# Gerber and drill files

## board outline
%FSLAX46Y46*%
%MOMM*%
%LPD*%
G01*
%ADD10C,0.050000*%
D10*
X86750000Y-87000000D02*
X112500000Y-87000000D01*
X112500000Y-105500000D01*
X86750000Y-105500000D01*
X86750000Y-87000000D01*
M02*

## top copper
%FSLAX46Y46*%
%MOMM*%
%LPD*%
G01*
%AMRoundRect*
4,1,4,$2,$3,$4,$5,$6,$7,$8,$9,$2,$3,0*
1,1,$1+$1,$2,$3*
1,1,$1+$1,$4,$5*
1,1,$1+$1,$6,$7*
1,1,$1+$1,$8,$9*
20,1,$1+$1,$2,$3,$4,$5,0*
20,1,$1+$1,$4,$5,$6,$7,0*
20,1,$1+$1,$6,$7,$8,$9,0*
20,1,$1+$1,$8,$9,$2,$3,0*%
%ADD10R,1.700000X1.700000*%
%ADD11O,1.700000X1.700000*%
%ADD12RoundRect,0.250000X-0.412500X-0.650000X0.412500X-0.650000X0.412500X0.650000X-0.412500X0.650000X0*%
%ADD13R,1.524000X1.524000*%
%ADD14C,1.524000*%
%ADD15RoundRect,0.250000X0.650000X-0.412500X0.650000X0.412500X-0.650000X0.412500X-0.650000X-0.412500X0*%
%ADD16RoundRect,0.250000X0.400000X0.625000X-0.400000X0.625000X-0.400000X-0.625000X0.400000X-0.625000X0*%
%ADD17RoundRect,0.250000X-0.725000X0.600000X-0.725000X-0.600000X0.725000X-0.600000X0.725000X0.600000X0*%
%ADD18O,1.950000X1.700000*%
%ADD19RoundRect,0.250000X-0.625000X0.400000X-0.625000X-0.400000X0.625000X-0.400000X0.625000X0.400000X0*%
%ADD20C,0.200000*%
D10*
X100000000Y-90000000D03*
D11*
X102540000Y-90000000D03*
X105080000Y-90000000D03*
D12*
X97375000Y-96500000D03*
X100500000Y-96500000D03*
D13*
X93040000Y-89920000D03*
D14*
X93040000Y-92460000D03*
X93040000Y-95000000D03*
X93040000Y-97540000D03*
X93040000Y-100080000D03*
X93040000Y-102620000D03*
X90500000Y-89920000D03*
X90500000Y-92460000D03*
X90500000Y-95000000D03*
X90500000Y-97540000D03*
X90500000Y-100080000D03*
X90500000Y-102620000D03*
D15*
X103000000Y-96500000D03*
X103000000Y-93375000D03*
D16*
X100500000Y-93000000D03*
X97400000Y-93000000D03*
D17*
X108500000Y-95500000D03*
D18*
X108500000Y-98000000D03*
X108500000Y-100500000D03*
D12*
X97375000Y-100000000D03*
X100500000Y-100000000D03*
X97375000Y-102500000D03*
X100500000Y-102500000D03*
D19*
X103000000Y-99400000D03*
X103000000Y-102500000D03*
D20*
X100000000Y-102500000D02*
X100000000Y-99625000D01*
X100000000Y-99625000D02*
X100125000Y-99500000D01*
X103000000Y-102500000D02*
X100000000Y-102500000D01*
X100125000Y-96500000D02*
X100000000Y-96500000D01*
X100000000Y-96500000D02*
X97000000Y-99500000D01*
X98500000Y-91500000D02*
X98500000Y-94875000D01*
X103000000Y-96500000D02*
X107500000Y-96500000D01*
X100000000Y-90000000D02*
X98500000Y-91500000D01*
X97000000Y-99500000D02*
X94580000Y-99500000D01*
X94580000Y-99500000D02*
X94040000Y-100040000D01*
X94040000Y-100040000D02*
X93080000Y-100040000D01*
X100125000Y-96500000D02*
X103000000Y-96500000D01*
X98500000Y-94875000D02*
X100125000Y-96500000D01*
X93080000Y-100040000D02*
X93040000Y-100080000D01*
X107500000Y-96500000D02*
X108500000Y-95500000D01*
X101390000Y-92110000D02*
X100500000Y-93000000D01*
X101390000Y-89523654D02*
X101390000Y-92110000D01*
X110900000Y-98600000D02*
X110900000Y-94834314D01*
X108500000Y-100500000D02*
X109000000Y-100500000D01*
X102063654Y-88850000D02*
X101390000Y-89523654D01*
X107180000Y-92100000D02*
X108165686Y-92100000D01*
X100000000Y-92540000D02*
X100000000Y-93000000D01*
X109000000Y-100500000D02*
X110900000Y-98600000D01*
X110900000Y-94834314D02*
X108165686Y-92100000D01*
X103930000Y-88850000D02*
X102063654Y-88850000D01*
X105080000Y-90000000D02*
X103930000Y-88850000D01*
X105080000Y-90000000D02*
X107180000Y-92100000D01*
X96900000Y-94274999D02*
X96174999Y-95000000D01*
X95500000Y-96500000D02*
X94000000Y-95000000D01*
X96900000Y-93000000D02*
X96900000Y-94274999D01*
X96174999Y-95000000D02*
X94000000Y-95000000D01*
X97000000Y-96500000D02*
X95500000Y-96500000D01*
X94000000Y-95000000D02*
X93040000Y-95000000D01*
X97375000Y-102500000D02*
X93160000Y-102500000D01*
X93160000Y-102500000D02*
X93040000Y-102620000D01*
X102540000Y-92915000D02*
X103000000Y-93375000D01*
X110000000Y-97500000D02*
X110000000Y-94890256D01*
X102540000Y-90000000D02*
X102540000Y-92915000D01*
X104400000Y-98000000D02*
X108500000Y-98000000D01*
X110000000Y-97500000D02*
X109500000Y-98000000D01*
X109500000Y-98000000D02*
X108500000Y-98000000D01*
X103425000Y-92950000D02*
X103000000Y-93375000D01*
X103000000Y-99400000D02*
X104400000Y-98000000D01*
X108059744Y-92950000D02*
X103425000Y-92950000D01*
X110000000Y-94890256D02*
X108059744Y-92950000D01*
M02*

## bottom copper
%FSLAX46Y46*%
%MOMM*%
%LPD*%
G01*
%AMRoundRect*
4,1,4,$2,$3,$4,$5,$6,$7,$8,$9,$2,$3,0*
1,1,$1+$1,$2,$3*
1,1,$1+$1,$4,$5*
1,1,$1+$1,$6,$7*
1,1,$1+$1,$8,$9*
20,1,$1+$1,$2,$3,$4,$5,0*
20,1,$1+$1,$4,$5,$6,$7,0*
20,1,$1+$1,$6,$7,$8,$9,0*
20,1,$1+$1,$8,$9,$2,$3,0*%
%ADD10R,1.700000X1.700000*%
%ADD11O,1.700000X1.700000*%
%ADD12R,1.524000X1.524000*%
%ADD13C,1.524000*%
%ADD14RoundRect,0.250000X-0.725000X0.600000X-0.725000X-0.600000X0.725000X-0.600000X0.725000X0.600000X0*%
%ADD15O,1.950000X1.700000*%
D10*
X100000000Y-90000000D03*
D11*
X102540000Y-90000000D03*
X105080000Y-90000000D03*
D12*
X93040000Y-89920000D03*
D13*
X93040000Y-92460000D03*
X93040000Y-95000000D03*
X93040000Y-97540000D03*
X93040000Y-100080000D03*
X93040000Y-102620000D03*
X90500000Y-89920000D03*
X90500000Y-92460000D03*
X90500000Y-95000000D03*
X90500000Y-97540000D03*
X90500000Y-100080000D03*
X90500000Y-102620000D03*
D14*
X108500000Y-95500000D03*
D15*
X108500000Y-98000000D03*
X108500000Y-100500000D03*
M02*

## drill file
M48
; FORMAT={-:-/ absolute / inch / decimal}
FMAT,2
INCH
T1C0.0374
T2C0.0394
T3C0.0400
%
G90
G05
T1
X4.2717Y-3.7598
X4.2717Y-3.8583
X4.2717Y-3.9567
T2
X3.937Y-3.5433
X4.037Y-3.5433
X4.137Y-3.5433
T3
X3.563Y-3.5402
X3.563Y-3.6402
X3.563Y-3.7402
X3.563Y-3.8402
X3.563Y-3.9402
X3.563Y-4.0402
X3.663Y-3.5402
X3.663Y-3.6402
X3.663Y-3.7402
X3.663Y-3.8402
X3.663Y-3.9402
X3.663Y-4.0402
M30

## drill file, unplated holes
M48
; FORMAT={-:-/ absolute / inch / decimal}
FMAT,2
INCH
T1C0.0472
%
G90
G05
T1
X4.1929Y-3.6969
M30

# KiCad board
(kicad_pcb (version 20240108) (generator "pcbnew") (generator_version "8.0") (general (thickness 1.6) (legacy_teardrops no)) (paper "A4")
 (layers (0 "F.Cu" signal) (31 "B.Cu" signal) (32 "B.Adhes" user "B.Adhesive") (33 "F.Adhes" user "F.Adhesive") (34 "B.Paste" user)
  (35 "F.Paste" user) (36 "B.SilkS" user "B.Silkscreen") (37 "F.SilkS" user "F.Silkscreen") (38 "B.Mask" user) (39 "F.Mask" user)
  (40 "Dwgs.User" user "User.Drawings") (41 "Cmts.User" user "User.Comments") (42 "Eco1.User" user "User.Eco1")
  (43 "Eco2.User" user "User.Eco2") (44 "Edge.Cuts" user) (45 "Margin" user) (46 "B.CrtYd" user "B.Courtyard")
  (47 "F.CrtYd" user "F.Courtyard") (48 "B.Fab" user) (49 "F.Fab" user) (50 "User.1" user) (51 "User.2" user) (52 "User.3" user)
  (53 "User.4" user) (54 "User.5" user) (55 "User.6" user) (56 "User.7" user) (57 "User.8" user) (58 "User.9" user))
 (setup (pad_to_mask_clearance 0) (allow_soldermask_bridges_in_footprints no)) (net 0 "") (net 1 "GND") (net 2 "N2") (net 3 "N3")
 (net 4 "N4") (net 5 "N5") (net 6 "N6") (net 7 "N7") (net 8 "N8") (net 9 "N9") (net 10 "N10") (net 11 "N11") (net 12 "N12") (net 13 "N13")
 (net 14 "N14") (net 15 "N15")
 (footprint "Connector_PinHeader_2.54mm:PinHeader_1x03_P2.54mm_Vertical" (layer "F.Cu") (at 100 90 90)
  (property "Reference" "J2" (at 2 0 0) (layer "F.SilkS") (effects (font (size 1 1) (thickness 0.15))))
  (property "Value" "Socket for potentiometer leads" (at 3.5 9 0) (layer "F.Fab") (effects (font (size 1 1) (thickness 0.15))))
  (pad "1" thru_hole rect (at 0 0 90) (size 1.7 1.7) (drill 1) (layers "*.Cu" "*.Mask") (remove_unused_layers no) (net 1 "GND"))
  (pad "2" thru_hole oval (at 0 2.54 90) (size 1.7 1.7) (drill 1) (layers "*.Cu" "*.Mask") (remove_unused_layers no) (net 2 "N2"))
  (pad "3" thru_hole oval (at 0 5.08 90) (size 1.7 1.7) (drill 1) (layers "*.Cu" "*.Mask") (remove_unused_layers no) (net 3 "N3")))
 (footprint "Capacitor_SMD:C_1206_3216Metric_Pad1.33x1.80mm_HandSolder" (layer "F.Cu") (at 98.9375 96.5)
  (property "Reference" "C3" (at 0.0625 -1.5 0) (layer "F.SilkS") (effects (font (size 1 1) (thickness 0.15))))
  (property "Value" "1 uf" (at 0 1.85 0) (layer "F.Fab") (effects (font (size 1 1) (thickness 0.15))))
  (pad "1" smd roundrect (at -1.5625 0) (size 1.325 1.8) (layers "F.Cu" "F.Paste" "F.Mask") (roundrect_rratio 0.188679) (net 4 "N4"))
  (pad "2" smd roundrect (at 1.5625 0) (size 1.325 1.8) (layers "F.Cu" "F.Paste" "F.Mask") (roundrect_rratio 0.188679) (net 1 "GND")))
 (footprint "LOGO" (layer "F.Cu") (at 109.5 90)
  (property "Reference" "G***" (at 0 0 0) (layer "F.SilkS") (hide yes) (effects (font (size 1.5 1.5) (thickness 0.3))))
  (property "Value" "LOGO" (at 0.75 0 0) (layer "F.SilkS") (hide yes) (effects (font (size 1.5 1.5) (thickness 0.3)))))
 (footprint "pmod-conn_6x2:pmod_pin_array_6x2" (layer "F.Cu") (at 91.77 96.27)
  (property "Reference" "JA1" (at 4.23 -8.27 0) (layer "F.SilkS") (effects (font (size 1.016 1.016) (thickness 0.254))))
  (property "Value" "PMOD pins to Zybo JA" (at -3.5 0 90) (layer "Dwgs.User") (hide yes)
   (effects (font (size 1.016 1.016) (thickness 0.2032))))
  (pad "1" thru_hole rect (at 1.27 -6.35) (size 1.524 1.524) (drill 1.016) (layers "*.Cu" "*.Mask" "F.SilkS") (remove_unused_layers no)
   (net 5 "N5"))
  (pad "2" thru_hole circle (at 1.27 -3.81 270) (size 1.524 1.524) (drill 1.016) (layers "*.Cu" "*.Mask" "F.SilkS")
   (remove_unused_layers no) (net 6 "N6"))
  (pad "3" thru_hole circle (at 1.27 -1.27 270) (size 1.524 1.524) (drill 1.016) (layers "*.Cu" "*.Mask" "F.SilkS")
   (remove_unused_layers no) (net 4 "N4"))
  (pad "4" thru_hole circle (at 1.27 1.27 270) (size 1.524 1.524) (drill 1.016) (layers "*.Cu" "*.Mask" "F.SilkS") (remove_unused_layers no)
   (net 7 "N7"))
  (pad "5" thru_hole circle (at 1.27 3.81 270) (size 1.524 1.524) (drill 1.016) (layers "*.Cu" "*.Mask" "F.SilkS") (remove_unused_layers no)
   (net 1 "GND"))
  (pad "6" thru_hole circle (at 1.27 6.35 270) (size 1.524 1.524) (drill 1.016) (layers "*.Cu" "*.Mask" "F.SilkS") (remove_unused_layers no)
   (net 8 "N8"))
  (pad "7" thru_hole circle (at -1.27 -6.35 270) (size 1.524 1.524) (drill 1.016) (layers "*.Cu" "*.Mask" "F.SilkS")
   (remove_unused_layers no) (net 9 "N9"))
  (pad "8" thru_hole circle (at -1.27 -3.81 270) (size 1.524 1.524) (drill 1.016) (layers "*.Cu" "*.Mask" "F.SilkS")
   (remove_unused_layers no) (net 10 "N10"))
  (pad "9" thru_hole circle (at -1.27 -1.27 270) (size 1.524 1.524) (drill 1.016) (layers "*.Cu" "*.Mask" "F.SilkS")
   (remove_unused_layers no) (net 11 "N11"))
  (pad "10" thru_hole circle (at -1.27 1.27 270) (size 1.524 1.524) (drill 1.016) (layers "*.Cu" "*.Mask" "F.SilkS")
   (remove_unused_layers no) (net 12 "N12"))
  (pad "11" thru_hole circle (at -1.27 3.81 270) (size 1.524 1.524) (drill 1.016) (layers "*.Cu" "*.Mask" "F.SilkS")
   (remove_unused_layers no) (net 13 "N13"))
  (pad "12" thru_hole circle (at -1.27 6.35 270) (size 1.524 1.524) (drill 1.016) (layers "*.Cu" "*.Mask" "F.SilkS")
   (remove_unused_layers no) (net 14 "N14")))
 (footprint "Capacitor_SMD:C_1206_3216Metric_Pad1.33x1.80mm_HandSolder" (layer "F.Cu") (at 103 94.9375 90)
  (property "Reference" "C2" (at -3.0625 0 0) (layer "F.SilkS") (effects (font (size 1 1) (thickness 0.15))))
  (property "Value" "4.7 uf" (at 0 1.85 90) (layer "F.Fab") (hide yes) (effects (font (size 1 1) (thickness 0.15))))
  (pad "1" smd roundrect (at -1.5625 0 90) (size 1.325 1.8) (layers "F.Cu" "F.Paste" "F.Mask") (roundrect_rratio 0.188679) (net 1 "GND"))
  (pad "2" smd roundrect (at 1.5625 0 90) (size 1.325 1.8) (layers "F.Cu" "F.Paste" "F.Mask") (roundrect_rratio 0.188679) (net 2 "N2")))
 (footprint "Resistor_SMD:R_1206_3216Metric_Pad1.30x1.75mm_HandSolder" (layer "F.Cu") (at 98.95 93 180)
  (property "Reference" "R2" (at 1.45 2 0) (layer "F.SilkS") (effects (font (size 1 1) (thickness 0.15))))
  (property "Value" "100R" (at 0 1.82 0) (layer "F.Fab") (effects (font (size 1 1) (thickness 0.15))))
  (pad "1" smd roundrect (at -1.55 0 180) (size 1.3 1.75) (layers "F.Cu" "F.Paste" "F.Mask") (roundrect_rratio 0.192308) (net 3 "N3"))
  (pad "2" smd roundrect (at 1.55 0 180) (size 1.3 1.75) (layers "F.Cu" "F.Paste" "F.Mask") (roundrect_rratio 0.192308) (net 4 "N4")))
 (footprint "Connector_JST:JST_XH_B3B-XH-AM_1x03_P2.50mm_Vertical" (layer "F.Cu") (at 108.5 95.5 -90)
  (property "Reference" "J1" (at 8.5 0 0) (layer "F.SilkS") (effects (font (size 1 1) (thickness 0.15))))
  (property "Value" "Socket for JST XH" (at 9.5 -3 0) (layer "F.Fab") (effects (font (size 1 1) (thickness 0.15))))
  (pad "" np_thru_hole circle (at -1.6 2 270) (size 1.2 1.2) (drill 1.2) (layers "*.Cu" "*.Mask"))
  (pad "1" thru_hole roundrect (at 0 0 270) (size 1.7 1.95) (drill 0.95) (layers "*.Cu" "*.Mask") (remove_unused_layers no)
   (roundrect_rratio 0.147059) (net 1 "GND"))
  (pad "2" thru_hole oval (at 2.5 0 270) (size 1.7 1.95) (drill 0.95) (layers "*.Cu" "*.Mask") (remove_unused_layers no) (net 2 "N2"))
  (pad "3" thru_hole oval (at 5 0 270) (size 1.7 1.95) (drill 0.95) (layers "*.Cu" "*.Mask") (remove_unused_layers no) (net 3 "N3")))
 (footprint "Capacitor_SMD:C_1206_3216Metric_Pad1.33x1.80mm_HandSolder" (layer "F.Cu") (at 98.9375 100)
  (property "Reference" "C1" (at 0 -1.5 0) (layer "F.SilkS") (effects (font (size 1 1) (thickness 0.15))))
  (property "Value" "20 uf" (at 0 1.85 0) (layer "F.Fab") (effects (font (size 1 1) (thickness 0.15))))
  (pad "1" smd roundrect (at -1.5625 0) (size 1.325 1.8) (layers "F.Cu" "F.Paste" "F.Mask") (roundrect_rratio 0.188679) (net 1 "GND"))
  (pad "2" smd roundrect (at 1.5625 0) (size 1.325 1.8) (layers "F.Cu" "F.Paste" "F.Mask") (roundrect_rratio 0.188679) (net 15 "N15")))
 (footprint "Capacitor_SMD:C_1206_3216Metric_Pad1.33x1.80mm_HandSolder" (layer "F.Cu") (at 98.9375 102.5)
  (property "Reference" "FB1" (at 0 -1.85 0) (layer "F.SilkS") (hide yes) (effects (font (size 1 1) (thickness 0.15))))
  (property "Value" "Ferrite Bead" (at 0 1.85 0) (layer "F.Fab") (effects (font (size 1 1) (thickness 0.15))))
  (pad "1" smd roundrect (at -1.5625 0) (size 1.325 1.8) (layers "F.Cu" "F.Paste" "F.Mask") (roundrect_rratio 0.188679) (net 8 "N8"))
  (pad "2" smd roundrect (at 1.5625 0) (size 1.325 1.8) (layers "F.Cu" "F.Paste" "F.Mask") (roundrect_rratio 0.188679) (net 15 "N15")))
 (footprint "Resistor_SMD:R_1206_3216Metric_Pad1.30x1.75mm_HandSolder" (layer "F.Cu") (at 103 100.95 -90)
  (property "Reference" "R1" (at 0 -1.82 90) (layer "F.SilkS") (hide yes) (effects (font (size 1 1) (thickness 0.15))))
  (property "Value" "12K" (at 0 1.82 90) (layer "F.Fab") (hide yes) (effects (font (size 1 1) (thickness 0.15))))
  (pad "1" smd roundrect (at -1.55 0 270) (size 1.3 1.75) (layers "F.Cu" "F.Paste" "F.Mask") (roundrect_rratio 0.192308) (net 2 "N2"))
  (pad "2" smd roundrect (at 1.55 0 270) (size 1.3 1.75) (layers "F.Cu" "F.Paste" "F.Mask") (roundrect_rratio 0.192308) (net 15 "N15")))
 (gr_rect (start 86.75 87) (end 112.5 105.5) (stroke (width 0.05) (type default)) (fill none) (layer "Edge.Cuts"))
 (segment (start 100 102.5) (end 100 99.625) (width 0.2) (layer "F.Cu") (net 15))
 (segment (start 100 99.625) (end 100.125 99.5) (width 0.2) (layer "F.Cu") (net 15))
 (segment (start 103 102.5) (end 100 102.5) (width 0.2) (layer "F.Cu") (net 15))
 (segment (start 100.125 96.5) (end 100 96.5) (width 0.2) (layer "F.Cu") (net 1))
 (segment (start 100 96.5) (end 97 99.5) (width 0.2) (layer "F.Cu") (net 1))
 (segment (start 98.5 91.5) (end 98.5 94.875) (width 0.2) (layer "F.Cu") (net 1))
 (segment (start 103 96.5) (end 107.5 96.5) (width 0.2) (layer "F.Cu") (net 1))
 (segment (start 100 90) (end 98.5 91.5) (width 0.2) (layer "F.Cu") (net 1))
 (segment (start 97 99.5) (end 94.58 99.5) (width 0.2) (layer "F.Cu") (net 1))
 (segment (start 94.58 99.5) (end 94.04 100.04) (width 0.2) (layer "F.Cu") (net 1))
 (segment (start 94.04 100.04) (end 93.08 100.04) (width 0.2) (layer "F.Cu") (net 1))
 (segment (start 100.125 96.5) (end 103 96.5) (width 0.2) (layer "F.Cu") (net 1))
 (segment (start 98.5 94.875) (end 100.125 96.5) (width 0.2) (layer "F.Cu") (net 1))
 (segment (start 93.08 100.04) (end 93.04 100.08) (width 0.2) (layer "F.Cu") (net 1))
 (segment (start 107.5 96.5) (end 108.5 95.5) (width 0.2) (layer "F.Cu") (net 1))
 (segment (start 101.39 92.11) (end 100.5 93) (width 0.2) (layer "F.Cu") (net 3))
 (segment (start 101.39 89.523654) (end 101.39 92.11) (width 0.2) (layer "F.Cu") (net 3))
 (segment (start 110.9 98.6) (end 110.9 94.834314) (width 0.2) (layer "F.Cu") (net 3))
 (segment (start 108.5 100.5) (end 109 100.5) (width 0.2) (layer "F.Cu") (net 3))
 (segment (start 102.063654 88.85) (end 101.39 89.523654) (width 0.2) (layer "F.Cu") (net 3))
 (segment (start 107.18 92.1) (end 108.165686 92.1) (width 0.2) (layer "F.Cu") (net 3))
 (segment (start 100 92.54) (end 100 93) (width 0.2) (layer "F.Cu") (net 3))
 (segment (start 109 100.5) (end 110.9 98.6) (width 0.2) (layer "F.Cu") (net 3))
 (segment (start 110.9 94.834314) (end 108.165686 92.1) (width 0.2) (layer "F.Cu") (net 3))
 (segment (start 103.93 88.85) (end 102.063654 88.85) (width 0.2) (layer "F.Cu") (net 3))
 (segment (start 105.08 90) (end 103.93 88.85) (width 0.2) (layer "F.Cu") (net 3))
 (segment (start 105.08 90) (end 107.18 92.1) (width 0.2) (layer "F.Cu") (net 3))
 (segment (start 96.9 94.274999) (end 96.174999 95) (width 0.2) (layer "F.Cu") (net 4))
 (segment (start 95.5 96.5) (end 94 95) (width 0.2) (layer "F.Cu") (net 4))
 (segment (start 96.9 93) (end 96.9 94.274999) (width 0.2) (layer "F.Cu") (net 4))
 (segment (start 96.174999 95) (end 94 95) (width 0.2) (layer "F.Cu") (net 4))
 (segment (start 97 96.5) (end 95.5 96.5) (width 0.2) (layer "F.Cu") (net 4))
 (segment (start 94 95) (end 93.04 95) (width 0.2) (layer "F.Cu") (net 4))
 (segment (start 97.375 102.5) (end 93.16 102.5) (width 0.2) (layer "F.Cu") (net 8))
 (segment (start 93.16 102.5) (end 93.04 102.62) (width 0.2) (layer "F.Cu") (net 8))
 (segment (start 102.54 92.915) (end 103 93.375) (width 0.2) (layer "F.Cu") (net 2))
 (segment (start 110 97.5) (end 110 94.890256) (width 0.2) (layer "F.Cu") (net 2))
 (segment (start 102.54 90) (end 102.54 92.915) (width 0.2) (layer "F.Cu") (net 2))
 (segment (start 104.4 98) (end 108.5 98) (width 0.2) (layer "F.Cu") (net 2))
 (segment (start 110 97.5) (end 109.5 98) (width 0.2) (layer "F.Cu") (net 2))
 (segment (start 109.5 98) (end 108.5 98) (width 0.2) (layer "F.Cu") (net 2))
 (segment (start 103.425 92.95) (end 103 93.375) (width 0.2) (layer "F.Cu") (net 2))
 (segment (start 103 99.4) (end 104.4 98) (width 0.2) (layer "F.Cu") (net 2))
 (segment (start 108.059744 92.95) (end 103.425 92.95) (width 0.2) (layer "F.Cu") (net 2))
 (segment (start 110 94.890256) (end 108.059744 92.95) (width 0.2) (layer "F.Cu") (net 2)))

